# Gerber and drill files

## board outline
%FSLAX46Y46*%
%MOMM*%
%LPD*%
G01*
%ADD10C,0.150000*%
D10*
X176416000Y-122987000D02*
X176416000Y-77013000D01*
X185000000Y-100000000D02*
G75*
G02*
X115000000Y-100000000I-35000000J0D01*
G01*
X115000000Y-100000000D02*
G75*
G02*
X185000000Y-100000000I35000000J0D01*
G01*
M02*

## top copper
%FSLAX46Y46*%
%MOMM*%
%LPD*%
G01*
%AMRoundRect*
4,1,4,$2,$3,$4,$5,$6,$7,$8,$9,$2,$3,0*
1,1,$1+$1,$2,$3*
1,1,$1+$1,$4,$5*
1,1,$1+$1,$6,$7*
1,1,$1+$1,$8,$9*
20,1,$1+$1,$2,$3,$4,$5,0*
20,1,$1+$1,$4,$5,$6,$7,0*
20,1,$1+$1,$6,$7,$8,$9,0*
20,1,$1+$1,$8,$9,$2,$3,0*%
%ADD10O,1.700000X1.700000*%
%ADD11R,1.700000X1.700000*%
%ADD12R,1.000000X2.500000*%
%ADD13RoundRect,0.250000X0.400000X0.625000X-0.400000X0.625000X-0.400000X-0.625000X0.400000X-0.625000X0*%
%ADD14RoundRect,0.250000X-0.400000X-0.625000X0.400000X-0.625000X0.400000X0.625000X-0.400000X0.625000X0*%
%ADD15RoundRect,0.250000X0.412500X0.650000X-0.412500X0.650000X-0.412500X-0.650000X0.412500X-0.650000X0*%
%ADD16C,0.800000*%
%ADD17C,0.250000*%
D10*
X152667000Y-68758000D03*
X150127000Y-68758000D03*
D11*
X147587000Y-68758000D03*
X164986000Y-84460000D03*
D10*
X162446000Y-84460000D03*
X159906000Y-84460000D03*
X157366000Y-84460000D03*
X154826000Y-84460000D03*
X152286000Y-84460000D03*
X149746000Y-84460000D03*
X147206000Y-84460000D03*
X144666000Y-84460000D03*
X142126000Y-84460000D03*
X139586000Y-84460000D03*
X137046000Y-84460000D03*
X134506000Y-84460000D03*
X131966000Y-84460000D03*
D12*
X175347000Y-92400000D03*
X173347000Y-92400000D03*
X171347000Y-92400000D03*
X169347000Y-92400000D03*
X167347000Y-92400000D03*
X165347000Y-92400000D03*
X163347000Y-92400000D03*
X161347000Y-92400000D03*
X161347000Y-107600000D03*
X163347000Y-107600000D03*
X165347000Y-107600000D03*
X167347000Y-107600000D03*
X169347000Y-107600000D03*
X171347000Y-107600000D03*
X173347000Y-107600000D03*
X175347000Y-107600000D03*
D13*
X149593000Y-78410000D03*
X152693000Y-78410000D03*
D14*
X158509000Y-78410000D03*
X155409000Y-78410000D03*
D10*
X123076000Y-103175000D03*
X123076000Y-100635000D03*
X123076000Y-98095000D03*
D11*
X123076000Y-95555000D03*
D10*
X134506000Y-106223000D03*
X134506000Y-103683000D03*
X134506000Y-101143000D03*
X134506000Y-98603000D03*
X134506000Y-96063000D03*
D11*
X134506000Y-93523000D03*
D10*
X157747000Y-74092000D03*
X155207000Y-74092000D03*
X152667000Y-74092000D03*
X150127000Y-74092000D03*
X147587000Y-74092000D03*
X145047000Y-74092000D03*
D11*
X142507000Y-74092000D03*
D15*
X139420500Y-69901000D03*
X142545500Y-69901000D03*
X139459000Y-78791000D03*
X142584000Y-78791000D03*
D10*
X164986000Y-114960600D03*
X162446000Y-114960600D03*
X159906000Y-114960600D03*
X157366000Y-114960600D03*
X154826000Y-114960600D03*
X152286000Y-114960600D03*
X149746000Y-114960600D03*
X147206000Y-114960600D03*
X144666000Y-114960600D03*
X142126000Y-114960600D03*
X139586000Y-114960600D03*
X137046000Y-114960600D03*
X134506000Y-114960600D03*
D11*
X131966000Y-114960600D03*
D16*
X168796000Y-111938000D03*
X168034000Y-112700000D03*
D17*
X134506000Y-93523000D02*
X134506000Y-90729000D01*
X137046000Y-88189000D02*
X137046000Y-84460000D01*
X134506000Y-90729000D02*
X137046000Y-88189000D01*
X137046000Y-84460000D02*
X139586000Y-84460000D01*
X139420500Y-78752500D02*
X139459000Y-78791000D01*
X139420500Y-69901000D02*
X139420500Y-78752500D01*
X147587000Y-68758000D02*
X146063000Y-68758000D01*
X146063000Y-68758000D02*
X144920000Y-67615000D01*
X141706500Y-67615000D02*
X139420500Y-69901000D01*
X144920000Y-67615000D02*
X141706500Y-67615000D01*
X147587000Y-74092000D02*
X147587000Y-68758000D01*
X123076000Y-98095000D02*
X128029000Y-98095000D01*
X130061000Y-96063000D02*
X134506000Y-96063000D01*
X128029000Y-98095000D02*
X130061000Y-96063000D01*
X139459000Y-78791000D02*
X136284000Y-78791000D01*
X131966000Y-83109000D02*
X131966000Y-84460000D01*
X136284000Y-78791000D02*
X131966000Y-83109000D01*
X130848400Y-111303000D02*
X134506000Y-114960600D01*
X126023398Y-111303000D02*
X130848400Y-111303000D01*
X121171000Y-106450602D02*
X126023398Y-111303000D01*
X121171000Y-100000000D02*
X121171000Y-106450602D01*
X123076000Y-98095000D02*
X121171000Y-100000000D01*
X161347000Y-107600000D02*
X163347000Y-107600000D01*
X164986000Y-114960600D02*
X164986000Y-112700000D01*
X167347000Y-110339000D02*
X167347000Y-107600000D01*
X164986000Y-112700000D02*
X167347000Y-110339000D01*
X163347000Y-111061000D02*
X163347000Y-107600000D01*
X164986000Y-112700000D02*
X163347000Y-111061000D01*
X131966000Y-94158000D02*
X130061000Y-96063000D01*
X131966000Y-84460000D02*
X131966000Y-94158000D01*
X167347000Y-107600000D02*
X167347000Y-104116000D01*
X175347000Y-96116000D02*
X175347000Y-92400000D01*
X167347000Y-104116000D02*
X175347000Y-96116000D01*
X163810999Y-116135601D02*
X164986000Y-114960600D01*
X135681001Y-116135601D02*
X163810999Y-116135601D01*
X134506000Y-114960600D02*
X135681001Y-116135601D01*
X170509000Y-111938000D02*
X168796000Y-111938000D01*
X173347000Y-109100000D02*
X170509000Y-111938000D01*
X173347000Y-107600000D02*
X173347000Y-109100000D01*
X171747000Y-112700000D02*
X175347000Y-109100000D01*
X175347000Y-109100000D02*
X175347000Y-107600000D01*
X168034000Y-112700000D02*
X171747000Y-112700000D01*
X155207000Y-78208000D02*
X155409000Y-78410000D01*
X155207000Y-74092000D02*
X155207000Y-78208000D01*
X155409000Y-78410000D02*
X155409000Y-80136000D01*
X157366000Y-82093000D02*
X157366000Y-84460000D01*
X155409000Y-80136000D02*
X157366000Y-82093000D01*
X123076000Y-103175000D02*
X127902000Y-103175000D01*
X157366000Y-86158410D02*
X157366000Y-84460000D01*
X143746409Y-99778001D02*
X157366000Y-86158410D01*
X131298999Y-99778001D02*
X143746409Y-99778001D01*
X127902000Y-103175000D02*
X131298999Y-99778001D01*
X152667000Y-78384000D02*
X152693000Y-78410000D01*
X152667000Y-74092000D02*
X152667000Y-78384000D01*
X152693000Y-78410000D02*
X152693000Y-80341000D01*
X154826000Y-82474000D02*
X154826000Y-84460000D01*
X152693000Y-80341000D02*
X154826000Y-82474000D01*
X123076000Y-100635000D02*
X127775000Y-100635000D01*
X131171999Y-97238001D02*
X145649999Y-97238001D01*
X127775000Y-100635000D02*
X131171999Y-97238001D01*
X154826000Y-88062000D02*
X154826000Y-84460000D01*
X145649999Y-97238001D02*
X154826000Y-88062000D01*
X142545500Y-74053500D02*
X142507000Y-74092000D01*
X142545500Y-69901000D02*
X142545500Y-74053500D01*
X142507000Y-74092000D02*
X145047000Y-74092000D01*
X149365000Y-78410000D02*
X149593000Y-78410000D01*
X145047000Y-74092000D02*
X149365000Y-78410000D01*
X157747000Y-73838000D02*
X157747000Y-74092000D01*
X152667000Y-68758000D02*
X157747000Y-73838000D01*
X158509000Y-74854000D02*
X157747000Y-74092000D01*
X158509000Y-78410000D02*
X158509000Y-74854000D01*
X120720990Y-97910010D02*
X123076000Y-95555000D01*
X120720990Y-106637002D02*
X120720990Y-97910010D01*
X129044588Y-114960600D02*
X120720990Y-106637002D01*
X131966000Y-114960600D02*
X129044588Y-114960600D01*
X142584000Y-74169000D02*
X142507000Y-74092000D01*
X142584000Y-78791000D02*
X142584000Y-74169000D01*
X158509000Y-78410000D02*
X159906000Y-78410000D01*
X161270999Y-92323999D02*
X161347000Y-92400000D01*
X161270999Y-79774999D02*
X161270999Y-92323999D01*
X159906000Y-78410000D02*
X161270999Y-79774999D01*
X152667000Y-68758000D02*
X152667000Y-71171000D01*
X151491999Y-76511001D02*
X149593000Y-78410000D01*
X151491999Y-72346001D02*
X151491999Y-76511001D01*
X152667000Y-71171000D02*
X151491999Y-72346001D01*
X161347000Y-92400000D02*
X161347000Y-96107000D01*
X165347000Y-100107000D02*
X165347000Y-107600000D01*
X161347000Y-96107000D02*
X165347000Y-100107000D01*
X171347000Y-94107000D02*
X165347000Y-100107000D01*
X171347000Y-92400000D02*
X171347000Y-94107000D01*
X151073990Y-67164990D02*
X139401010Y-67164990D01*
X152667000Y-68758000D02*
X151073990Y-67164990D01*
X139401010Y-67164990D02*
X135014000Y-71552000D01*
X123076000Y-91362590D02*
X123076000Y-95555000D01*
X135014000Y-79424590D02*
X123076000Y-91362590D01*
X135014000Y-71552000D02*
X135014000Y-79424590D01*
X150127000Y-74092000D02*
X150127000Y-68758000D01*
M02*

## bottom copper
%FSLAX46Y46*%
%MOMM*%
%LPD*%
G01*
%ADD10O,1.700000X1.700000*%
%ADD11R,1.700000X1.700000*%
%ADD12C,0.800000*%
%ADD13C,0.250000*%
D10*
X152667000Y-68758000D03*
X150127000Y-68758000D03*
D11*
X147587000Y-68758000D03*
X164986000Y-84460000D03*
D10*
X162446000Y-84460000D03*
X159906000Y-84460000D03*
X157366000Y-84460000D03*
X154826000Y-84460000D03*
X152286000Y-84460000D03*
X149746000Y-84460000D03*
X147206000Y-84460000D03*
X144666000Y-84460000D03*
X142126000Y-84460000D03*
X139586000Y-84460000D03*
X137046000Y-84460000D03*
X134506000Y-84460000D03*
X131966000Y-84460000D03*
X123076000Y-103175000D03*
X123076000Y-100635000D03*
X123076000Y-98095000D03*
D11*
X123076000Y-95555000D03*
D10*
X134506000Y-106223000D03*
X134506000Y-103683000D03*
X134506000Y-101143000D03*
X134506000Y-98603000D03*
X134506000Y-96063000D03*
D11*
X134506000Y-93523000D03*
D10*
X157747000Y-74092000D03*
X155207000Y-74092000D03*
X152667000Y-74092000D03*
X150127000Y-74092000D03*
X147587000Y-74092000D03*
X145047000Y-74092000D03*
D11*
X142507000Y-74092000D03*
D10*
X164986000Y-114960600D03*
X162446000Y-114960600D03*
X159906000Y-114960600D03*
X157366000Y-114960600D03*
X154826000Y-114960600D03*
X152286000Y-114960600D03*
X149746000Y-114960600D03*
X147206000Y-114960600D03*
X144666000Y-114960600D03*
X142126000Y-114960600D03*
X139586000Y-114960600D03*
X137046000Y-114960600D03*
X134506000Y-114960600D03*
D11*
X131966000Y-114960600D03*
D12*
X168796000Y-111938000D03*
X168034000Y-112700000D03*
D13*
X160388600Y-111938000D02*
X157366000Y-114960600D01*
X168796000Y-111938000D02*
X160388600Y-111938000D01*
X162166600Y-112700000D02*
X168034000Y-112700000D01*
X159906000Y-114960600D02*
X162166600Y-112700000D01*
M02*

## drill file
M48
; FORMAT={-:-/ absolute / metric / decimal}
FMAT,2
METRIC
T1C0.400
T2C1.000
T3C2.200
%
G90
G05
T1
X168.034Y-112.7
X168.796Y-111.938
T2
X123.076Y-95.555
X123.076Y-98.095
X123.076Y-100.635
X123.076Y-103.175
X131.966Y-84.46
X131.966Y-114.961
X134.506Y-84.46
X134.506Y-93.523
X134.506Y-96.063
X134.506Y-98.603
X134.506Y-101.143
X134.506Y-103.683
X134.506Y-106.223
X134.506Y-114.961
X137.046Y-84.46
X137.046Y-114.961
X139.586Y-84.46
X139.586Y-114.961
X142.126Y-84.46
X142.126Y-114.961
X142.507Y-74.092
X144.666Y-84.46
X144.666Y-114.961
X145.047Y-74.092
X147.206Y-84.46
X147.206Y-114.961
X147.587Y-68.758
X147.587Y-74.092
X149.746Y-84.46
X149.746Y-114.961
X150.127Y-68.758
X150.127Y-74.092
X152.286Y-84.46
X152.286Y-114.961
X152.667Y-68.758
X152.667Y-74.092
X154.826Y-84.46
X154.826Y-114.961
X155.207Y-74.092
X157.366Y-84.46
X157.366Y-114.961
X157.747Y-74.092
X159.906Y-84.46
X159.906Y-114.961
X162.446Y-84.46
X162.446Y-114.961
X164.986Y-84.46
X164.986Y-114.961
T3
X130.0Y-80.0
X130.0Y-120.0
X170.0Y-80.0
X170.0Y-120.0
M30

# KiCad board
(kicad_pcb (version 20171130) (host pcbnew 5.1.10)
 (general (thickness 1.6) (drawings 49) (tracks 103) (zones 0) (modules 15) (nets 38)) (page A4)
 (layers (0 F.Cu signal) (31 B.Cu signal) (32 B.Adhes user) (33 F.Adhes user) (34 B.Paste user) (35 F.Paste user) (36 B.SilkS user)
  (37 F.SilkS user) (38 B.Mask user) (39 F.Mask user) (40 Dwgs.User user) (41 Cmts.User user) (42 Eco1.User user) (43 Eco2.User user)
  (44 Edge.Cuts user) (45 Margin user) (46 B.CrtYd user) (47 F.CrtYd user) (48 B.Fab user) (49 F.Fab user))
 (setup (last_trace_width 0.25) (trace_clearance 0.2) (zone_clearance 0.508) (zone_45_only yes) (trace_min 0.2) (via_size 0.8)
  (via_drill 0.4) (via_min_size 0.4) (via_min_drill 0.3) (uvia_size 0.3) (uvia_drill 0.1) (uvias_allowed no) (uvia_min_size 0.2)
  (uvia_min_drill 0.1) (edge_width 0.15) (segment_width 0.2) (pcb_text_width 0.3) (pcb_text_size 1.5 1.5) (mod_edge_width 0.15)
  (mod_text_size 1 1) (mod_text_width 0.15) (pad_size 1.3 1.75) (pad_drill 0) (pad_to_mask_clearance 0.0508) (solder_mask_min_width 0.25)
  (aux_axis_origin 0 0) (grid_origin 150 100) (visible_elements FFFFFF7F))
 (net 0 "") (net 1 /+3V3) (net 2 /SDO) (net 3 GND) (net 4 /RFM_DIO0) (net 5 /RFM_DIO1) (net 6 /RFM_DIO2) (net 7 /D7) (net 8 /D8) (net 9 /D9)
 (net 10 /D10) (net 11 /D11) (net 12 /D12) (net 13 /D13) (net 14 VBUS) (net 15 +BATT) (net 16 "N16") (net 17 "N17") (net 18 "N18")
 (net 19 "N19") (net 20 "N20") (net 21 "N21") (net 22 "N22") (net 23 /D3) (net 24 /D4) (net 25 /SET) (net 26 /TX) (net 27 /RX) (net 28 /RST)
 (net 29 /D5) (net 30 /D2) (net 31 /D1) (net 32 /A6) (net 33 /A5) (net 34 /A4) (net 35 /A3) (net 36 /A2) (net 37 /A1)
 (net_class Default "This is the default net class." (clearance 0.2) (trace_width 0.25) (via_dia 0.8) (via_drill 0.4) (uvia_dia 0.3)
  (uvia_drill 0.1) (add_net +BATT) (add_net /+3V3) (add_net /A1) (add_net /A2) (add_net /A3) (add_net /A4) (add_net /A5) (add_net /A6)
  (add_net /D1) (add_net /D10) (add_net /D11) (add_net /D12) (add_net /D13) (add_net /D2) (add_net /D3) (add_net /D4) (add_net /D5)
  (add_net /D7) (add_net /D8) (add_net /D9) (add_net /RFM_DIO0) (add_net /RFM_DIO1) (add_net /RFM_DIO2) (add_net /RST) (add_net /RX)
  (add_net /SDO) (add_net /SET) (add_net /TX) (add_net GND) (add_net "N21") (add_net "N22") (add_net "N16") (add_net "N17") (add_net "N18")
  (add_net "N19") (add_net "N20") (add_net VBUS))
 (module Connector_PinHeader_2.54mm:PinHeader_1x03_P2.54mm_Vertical (layer F.Cu) (at 147.587 68.758 90)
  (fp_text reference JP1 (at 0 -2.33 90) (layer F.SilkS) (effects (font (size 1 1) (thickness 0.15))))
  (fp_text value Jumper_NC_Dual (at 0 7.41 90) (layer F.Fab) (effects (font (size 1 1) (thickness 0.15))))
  (pad 3 thru_hole oval (at 0 5.08 90) (size 1.7 1.7) (drill 1) (layers *.Cu *.Mask) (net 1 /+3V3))
  (pad 2 thru_hole oval (at 0 2.54 90) (size 1.7 1.7) (drill 1) (layers *.Cu *.Mask) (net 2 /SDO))
  (pad 1 thru_hole rect (at 0 0 90) (size 1.7 1.7) (drill 1) (layers *.Cu *.Mask) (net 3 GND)))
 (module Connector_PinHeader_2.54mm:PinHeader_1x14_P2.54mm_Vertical (layer F.Cu) (at 164.986 84.46 270)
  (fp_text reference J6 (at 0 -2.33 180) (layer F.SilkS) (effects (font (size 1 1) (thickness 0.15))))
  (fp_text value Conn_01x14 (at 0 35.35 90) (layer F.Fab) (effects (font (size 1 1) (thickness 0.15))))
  (pad 1 thru_hole rect (at 0 0 270) (size 1.7 1.7) (drill 1) (layers *.Cu *.Mask) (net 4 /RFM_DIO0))
  (pad 2 thru_hole oval (at 0 2.54 270) (size 1.7 1.7) (drill 1) (layers *.Cu *.Mask) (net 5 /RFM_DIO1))
  (pad 3 thru_hole oval (at 0 5.08 270) (size 1.7 1.7) (drill 1) (layers *.Cu *.Mask) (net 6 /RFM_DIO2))
  (pad 4 thru_hole oval (at 0 7.62 270) (size 1.7 1.7) (drill 1) (layers *.Cu *.Mask) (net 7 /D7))
  (pad 5 thru_hole oval (at 0 10.16 270) (size 1.7 1.7) (drill 1) (layers *.Cu *.Mask) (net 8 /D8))
  (pad 6 thru_hole oval (at 0 12.7 270) (size 1.7 1.7) (drill 1) (layers *.Cu *.Mask) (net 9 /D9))
  (pad 7 thru_hole oval (at 0 15.24 270) (size 1.7 1.7) (drill 1) (layers *.Cu *.Mask) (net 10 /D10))
  (pad 8 thru_hole oval (at 0 17.78 270) (size 1.7 1.7) (drill 1) (layers *.Cu *.Mask) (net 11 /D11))
  (pad 9 thru_hole oval (at 0 20.32 270) (size 1.7 1.7) (drill 1) (layers *.Cu *.Mask) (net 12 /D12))
  (pad 10 thru_hole oval (at 0 22.86 270) (size 1.7 1.7) (drill 1) (layers *.Cu *.Mask) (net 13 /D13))
  (pad 11 thru_hole oval (at 0 25.4 270) (size 1.7 1.7) (drill 1) (layers *.Cu *.Mask) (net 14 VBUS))
  (pad 12 thru_hole oval (at 0 27.94 270) (size 1.7 1.7) (drill 1) (layers *.Cu *.Mask) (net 14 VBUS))
  (pad 13 thru_hole oval (at 0 30.48 270) (size 1.7 1.7) (drill 1) (layers *.Cu *.Mask) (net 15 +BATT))
  (pad 14 thru_hole oval (at 0 33.02 270) (size 1.7 1.7) (drill 1) (layers *.Cu *.Mask) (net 3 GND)))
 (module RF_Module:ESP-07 (layer F.Cu) (at 170.447 100 270)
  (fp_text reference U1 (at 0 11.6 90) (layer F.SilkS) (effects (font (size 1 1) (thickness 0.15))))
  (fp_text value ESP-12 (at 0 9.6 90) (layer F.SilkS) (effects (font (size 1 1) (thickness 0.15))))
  (pad 1 smd rect (at -7.6 -4.9 270) (size 2.5 1) (layers F.Cu F.Paste F.Mask) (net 3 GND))
  (pad 2 smd rect (at -7.6 -2.9 270) (size 2.5 1) (layers F.Cu F.Paste F.Mask) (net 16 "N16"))
  (pad 3 smd rect (at -7.6 -0.9 270) (size 2.5 1) (layers F.Cu F.Paste F.Mask) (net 1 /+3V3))
  (pad 4 smd rect (at -7.6 1.1 270) (size 2.5 1) (layers F.Cu F.Paste F.Mask) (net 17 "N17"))
  (pad 5 smd rect (at -7.6 3.1 270) (size 2.5 1) (layers F.Cu F.Paste F.Mask) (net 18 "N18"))
  (pad 6 smd rect (at -7.6 5.1 270) (size 2.5 1) (layers F.Cu F.Paste F.Mask) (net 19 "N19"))
  (pad 7 smd rect (at -7.6 7.1 270) (size 2.5 1) (layers F.Cu F.Paste F.Mask) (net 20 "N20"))
  (pad 8 smd rect (at -7.6 9.1 270) (size 2.5 1) (layers F.Cu F.Paste F.Mask) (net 1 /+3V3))
  (pad 9 smd rect (at 7.6 9.1 270) (size 2.5 1) (layers F.Cu F.Paste F.Mask) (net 3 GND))
  (pad 10 smd rect (at 7.6 7.1 270) (size 2.5 1) (layers F.Cu F.Paste F.Mask) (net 3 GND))
  (pad 11 smd rect (at 7.6 5.1 270) (size 2.5 1) (layers F.Cu F.Paste F.Mask) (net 1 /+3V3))
  (pad 12 smd rect (at 7.6 3.1 270) (size 2.5 1) (layers F.Cu F.Paste F.Mask) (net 3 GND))
  (pad 13 smd rect (at 7.6 1.1 270) (size 2.5 1) (layers F.Cu F.Paste F.Mask) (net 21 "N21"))
  (pad 14 smd rect (at 7.6 -0.9 270) (size 2.5 1) (layers F.Cu F.Paste F.Mask) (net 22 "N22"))
  (pad 15 smd rect (at 7.6 -2.9 270) (size 2.5 1) (layers F.Cu F.Paste F.Mask) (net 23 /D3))
  (pad 16 smd rect (at 7.6 -4.9 270) (size 2.5 1) (layers F.Cu F.Paste F.Mask) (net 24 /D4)))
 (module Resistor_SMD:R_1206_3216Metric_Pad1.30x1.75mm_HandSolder (layer F.Cu) (at 151.143 78.41 180)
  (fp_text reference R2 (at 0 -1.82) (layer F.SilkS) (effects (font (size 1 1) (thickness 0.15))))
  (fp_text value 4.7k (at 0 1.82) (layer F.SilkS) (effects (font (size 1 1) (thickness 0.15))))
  (pad 2 smd roundrect (at 1.55 0 180) (size 1.3 1.75) (layers F.Cu F.Paste F.Mask) (roundrect_rratio 0.192308) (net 1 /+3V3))
  (pad 1 smd roundrect (at -1.55 0 180) (size 1.3 1.75) (layers F.Cu F.Paste F.Mask) (roundrect_rratio 0.192308) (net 8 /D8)))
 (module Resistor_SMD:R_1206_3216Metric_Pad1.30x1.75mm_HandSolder (layer F.Cu) (at 156.959 78.41)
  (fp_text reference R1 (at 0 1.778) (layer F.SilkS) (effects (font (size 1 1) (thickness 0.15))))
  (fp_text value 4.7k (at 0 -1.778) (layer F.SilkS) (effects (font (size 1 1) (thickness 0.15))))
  (pad 2 smd roundrect (at 1.55 0) (size 1.3 1.75) (layers F.Cu F.Paste F.Mask) (roundrect_rratio 0.192308) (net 1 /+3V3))
  (pad 1 smd roundrect (at -1.55 0) (size 1.3 1.75) (layers F.Cu F.Paste F.Mask) (roundrect_rratio 0.192308) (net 7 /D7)))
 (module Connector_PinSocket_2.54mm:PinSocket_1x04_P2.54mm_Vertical (layer F.Cu) (at 123.076 95.555)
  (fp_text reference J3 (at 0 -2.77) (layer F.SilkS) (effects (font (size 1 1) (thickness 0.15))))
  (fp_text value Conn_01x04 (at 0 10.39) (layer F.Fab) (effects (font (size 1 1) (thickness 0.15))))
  (pad 4 thru_hole oval (at 0 7.62) (size 1.7 1.7) (drill 1) (layers *.Cu *.Mask) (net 7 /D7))
  (pad 3 thru_hole oval (at 0 5.08) (size 1.7 1.7) (drill 1) (layers *.Cu *.Mask) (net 8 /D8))
  (pad 2 thru_hole oval (at 0 2.54) (size 1.7 1.7) (drill 1) (layers *.Cu *.Mask) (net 3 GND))
  (pad 1 thru_hole rect (at 0 0) (size 1.7 1.7) (drill 1) (layers *.Cu *.Mask) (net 1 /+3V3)))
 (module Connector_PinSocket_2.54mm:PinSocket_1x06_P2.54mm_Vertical (layer F.Cu) (at 134.506 93.523)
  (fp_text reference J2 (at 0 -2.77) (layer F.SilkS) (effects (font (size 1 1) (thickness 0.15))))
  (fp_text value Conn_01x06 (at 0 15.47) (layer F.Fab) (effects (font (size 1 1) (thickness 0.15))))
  (pad 6 thru_hole oval (at 0 12.7) (size 1.7 1.7) (drill 1) (layers *.Cu *.Mask) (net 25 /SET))
  (pad 5 thru_hole oval (at 0 10.16) (size 1.7 1.7) (drill 1) (layers *.Cu *.Mask) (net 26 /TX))
  (pad 4 thru_hole oval (at 0 7.62) (size 1.7 1.7) (drill 1) (layers *.Cu *.Mask) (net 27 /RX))
  (pad 3 thru_hole oval (at 0 5.08) (size 1.7 1.7) (drill 1) (layers *.Cu *.Mask) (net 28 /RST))
  (pad 2 thru_hole oval (at 0 2.54) (size 1.7 1.7) (drill 1) (layers *.Cu *.Mask) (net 3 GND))
  (pad 1 thru_hole rect (at 0 0) (size 1.7 1.7) (drill 1) (layers *.Cu *.Mask) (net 14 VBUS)))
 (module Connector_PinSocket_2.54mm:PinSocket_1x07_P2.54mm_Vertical (layer F.Cu) (at 142.507 74.092 90)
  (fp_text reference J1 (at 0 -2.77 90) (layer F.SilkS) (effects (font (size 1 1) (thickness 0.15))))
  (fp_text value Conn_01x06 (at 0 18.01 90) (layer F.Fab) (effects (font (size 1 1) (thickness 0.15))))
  (pad 7 thru_hole oval (at 0 15.24 90) (size 1.7 1.7) (drill 1) (layers *.Cu *.Mask) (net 1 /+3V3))
  (pad 6 thru_hole oval (at 0 12.7 90) (size 1.7 1.7) (drill 1) (layers *.Cu *.Mask) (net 7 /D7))
  (pad 5 thru_hole oval (at 0 10.16 90) (size 1.7 1.7) (drill 1) (layers *.Cu *.Mask) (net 8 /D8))
  (pad 4 thru_hole oval (at 0 7.62 90) (size 1.7 1.7) (drill 1) (layers *.Cu *.Mask) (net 2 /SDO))
  (pad 3 thru_hole oval (at 0 5.08 90) (size 1.7 1.7) (drill 1) (layers *.Cu *.Mask) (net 3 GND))
  (pad 2 thru_hole oval (at 0 2.54 90) (size 1.7 1.7) (drill 1) (layers *.Cu *.Mask) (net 1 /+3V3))
  (pad 1 thru_hole rect (at 0 0 90) (size 1.7 1.7) (drill 1) (layers *.Cu *.Mask) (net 1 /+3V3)))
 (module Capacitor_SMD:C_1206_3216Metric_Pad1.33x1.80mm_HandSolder (layer F.Cu) (at 140.983 69.901 180)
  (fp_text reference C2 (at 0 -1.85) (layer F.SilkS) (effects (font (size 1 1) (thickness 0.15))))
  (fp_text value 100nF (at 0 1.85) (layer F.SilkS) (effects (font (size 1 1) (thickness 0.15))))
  (pad 2 smd roundrect (at 1.5625 0 180) (size 1.325 1.8) (layers F.Cu F.Paste F.Mask) (roundrect_rratio 0.188679) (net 3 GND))
  (pad 1 smd roundrect (at -1.5625 0 180) (size 1.325 1.8) (layers F.Cu F.Paste F.Mask) (roundrect_rratio 0.188679) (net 1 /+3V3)))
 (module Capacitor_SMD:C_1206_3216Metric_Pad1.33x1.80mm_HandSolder (layer F.Cu) (at 141.0215 78.791 180)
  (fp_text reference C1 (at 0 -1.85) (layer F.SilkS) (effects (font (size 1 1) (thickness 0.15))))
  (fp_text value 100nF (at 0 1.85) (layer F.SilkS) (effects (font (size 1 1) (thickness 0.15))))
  (pad 2 smd roundrect (at 1.5625 0 180) (size 1.325 1.8) (layers F.Cu F.Paste F.Mask) (roundrect_rratio 0.188679) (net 3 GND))
  (pad 1 smd roundrect (at -1.5625 0 180) (size 1.325 1.8) (layers F.Cu F.Paste F.Mask) (roundrect_rratio 0.188679) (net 1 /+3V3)))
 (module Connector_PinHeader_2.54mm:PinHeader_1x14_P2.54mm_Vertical (layer F.Cu) (at 131.966 114.9606 90)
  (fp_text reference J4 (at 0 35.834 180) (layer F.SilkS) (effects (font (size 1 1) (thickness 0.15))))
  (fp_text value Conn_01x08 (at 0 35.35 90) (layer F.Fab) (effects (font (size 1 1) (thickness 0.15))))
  (pad 14 thru_hole oval (at 0 33.02 90) (size 1.7 1.7) (drill 1) (layers *.Cu *.Mask) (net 3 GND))
  (pad 13 thru_hole oval (at 0 30.48 90) (size 1.7 1.7) (drill 1) (layers *.Cu *.Mask) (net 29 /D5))
  (pad 12 thru_hole oval (at 0 27.94 90) (size 1.7 1.7) (drill 1) (layers *.Cu *.Mask) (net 24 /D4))
  (pad 11 thru_hole oval (at 0 25.4 90) (size 1.7 1.7) (drill 1) (layers *.Cu *.Mask) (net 23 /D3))
  (pad 10 thru_hole oval (at 0 22.86 90) (size 1.7 1.7) (drill 1) (layers *.Cu *.Mask) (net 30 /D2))
  (pad 9 thru_hole oval (at 0 20.32 90) (size 1.7 1.7) (drill 1) (layers *.Cu *.Mask) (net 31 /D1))
  (pad 8 thru_hole oval (at 0 17.78 90) (size 1.7 1.7) (drill 1) (layers *.Cu *.Mask) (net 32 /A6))
  (pad 7 thru_hole oval (at 0 15.24 90) (size 1.7 1.7) (drill 1) (layers *.Cu *.Mask) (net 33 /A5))
  (pad 6 thru_hole oval (at 0 12.7 90) (size 1.7 1.7) (drill 1) (layers *.Cu *.Mask) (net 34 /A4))
  (pad 5 thru_hole oval (at 0 10.16 90) (size 1.7 1.7) (drill 1) (layers *.Cu *.Mask) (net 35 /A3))
  (pad 4 thru_hole oval (at 0 7.62 90) (size 1.7 1.7) (drill 1) (layers *.Cu *.Mask) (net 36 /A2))
  (pad 3 thru_hole oval (at 0 5.08 90) (size 1.7 1.7) (drill 1) (layers *.Cu *.Mask) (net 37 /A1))
  (pad 2 thru_hole oval (at 0 2.54 90) (size 1.7 1.7) (drill 1) (layers *.Cu *.Mask) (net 3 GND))
  (pad 1 thru_hole rect (at 0 0 90) (size 1.7 1.7) (drill 1) (layers *.Cu *.Mask) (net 1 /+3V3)))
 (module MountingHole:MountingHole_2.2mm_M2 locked (layer F.Cu) (at 130 120)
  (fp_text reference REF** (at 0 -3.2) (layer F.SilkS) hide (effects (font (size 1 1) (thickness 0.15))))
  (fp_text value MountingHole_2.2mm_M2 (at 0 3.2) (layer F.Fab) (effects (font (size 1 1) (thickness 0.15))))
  (pad 1 np_thru_hole circle (at 0 0) (size 2.2 2.2) (drill 2.2) (layers *.Cu *.Mask)))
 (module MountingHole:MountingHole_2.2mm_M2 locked (layer F.Cu) (at 170 120)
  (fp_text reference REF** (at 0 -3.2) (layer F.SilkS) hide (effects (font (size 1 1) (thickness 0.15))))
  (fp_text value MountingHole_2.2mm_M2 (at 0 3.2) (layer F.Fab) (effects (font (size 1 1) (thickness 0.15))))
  (pad 1 np_thru_hole circle (at 0 0) (size 2.2 2.2) (drill 2.2) (layers *.Cu *.Mask)))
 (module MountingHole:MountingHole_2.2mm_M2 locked (layer F.Cu) (at 130 80)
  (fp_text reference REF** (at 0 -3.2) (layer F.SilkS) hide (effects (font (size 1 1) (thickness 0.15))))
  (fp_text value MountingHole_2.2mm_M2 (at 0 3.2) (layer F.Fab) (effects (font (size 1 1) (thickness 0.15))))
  (pad 1 np_thru_hole circle (at 0 0) (size 2.2 2.2) (drill 2.2) (layers *.Cu *.Mask)))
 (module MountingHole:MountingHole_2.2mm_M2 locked (layer F.Cu) (at 170 80)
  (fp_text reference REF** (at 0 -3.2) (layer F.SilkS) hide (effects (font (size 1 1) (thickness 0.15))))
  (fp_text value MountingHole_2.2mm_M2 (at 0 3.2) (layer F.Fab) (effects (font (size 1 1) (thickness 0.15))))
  (pad 1 np_thru_hole circle (at 0 0) (size 2.2 2.2) (drill 2.2) (layers *.Cu *.Mask)))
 (gr_line (start 176.416 122.987) (end 176.416 77.013) (layer Edge.Cuts) (width 0.15))
 (gr_circle (center 150 100) (end 185 100) (layer Edge.Cuts) (width 0.15))
 (segment (start 134.506 93.523) (end 134.506 90.729) (width 0.25) (layer F.Cu) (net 14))
 (segment (start 137.046 88.189) (end 137.046 84.46) (width 0.25) (layer F.Cu) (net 14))
 (segment (start 134.506 90.729) (end 137.046 88.189) (width 0.25) (layer F.Cu) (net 14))
 (segment (start 137.046 84.46) (end 139.586 84.46) (width 0.25) (layer F.Cu) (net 14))
 (segment (start 139.4205 78.7525) (end 139.459 78.791) (width 0.25) (layer F.Cu) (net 3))
 (segment (start 139.4205 69.901) (end 139.4205 78.7525) (width 0.25) (layer F.Cu) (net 3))
 (segment (start 147.587 68.758) (end 146.063 68.758) (width 0.25) (layer F.Cu) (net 3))
 (segment (start 146.063 68.758) (end 144.92 67.615) (width 0.25) (layer F.Cu) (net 3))
 (segment (start 141.7065 67.615) (end 139.4205 69.901) (width 0.25) (layer F.Cu) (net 3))
 (segment (start 144.92 67.615) (end 141.7065 67.615) (width 0.25) (layer F.Cu) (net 3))
 (segment (start 147.587 74.092) (end 147.587 68.758) (width 0.25) (layer F.Cu) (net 3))
 (segment (start 123.076 98.095) (end 128.029 98.095) (width 0.25) (layer F.Cu) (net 3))
 (segment (start 130.061 96.063) (end 134.506 96.063) (width 0.25) (layer F.Cu) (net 3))
 (segment (start 128.029 98.095) (end 130.061 96.063) (width 0.25) (layer F.Cu) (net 3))
 (segment (start 139.459 78.791) (end 136.284 78.791) (width 0.25) (layer F.Cu) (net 3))
 (segment (start 131.966 83.109) (end 131.966 84.46) (width 0.25) (layer F.Cu) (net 3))
 (segment (start 136.284 78.791) (end 131.966 83.109) (width 0.25) (layer F.Cu) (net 3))
 (segment (start 130.8484 111.303) (end 134.506 114.9606) (width 0.25) (layer F.Cu) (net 3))
 (segment (start 126.023398 111.303) (end 130.8484 111.303) (width 0.25) (layer F.Cu) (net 3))
 (segment (start 121.171 106.450602) (end 126.023398 111.303) (width 0.25) (layer F.Cu) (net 3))
 (segment (start 121.171 100) (end 121.171 106.450602) (width 0.25) (layer F.Cu) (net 3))
 (segment (start 123.076 98.095) (end 121.171 100) (width 0.25) (layer F.Cu) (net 3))
 (segment (start 161.347 107.6) (end 163.347 107.6) (width 0.25) (layer F.Cu) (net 3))
 (segment (start 164.986 114.9606) (end 164.986 112.7) (width 0.25) (layer F.Cu) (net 3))
 (segment (start 167.347 110.339) (end 167.347 107.6) (width 0.25) (layer F.Cu) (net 3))
 (segment (start 164.986 112.7) (end 167.347 110.339) (width 0.25) (layer F.Cu) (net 3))
 (segment (start 163.347 111.061) (end 163.347 107.6) (width 0.25) (layer F.Cu) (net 3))
 (segment (start 164.986 112.7) (end 163.347 111.061) (width 0.25) (layer F.Cu) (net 3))
 (segment (start 131.966 94.158) (end 130.061 96.063) (width 0.25) (layer F.Cu) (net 3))
 (segment (start 131.966 84.46) (end 131.966 94.158) (width 0.25) (layer F.Cu) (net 3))
 (segment (start 167.347 107.6) (end 167.347 104.116) (width 0.25) (layer F.Cu) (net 3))
 (segment (start 175.347 96.116) (end 175.347 92.4) (width 0.25) (layer F.Cu) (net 3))
 (segment (start 167.347 104.116) (end 175.347 96.116) (width 0.25) (layer F.Cu) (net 3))
 (segment (start 163.810999 116.135601) (end 164.986 114.9606) (width 0.25) (layer F.Cu) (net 3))
 (segment (start 135.681001 116.135601) (end 163.810999 116.135601) (width 0.25) (layer F.Cu) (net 3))
 (segment (start 134.506 114.9606) (end 135.681001 116.135601) (width 0.25) (layer F.Cu) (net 3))
 (via (at 168.796 111.938) (size 0.8) (drill 0.4) (layers F.Cu B.Cu) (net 23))
 (segment (start 170.509 111.938) (end 168.796 111.938) (width 0.25) (layer F.Cu) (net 23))
 (segment (start 173.347 109.1) (end 170.509 111.938) (width 0.25) (layer F.Cu) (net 23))
 (segment (start 173.347 107.6) (end 173.347 109.1) (width 0.25) (layer F.Cu) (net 23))
 (segment (start 160.3886 111.938) (end 157.366 114.9606) (width 0.25) (layer B.Cu) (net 23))
 (segment (start 168.796 111.938) (end 160.3886 111.938) (width 0.25) (layer B.Cu) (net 23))
 (via (at 168.034 112.7) (size 0.8) (drill 0.4) (layers F.Cu B.Cu) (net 24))
 (segment (start 162.1666 112.7) (end 168.034 112.7) (width 0.25) (layer B.Cu) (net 24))
 (segment (start 159.906 114.9606) (end 162.1666 112.7) (width 0.25) (layer B.Cu) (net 24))
 (segment (start 171.747 112.7) (end 175.347 109.1) (width 0.25) (layer F.Cu) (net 24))
 (segment (start 175.347 109.1) (end 175.347 107.6) (width 0.25) (layer F.Cu) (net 24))
 (segment (start 168.034 112.7) (end 171.747 112.7) (width 0.25) (layer F.Cu) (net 24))
 (segment (start 155.207 78.208) (end 155.409 78.41) (width 0.25) (layer F.Cu) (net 7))
 (segment (start 155.207 74.092) (end 155.207 78.208) (width 0.25) (layer F.Cu) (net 7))
 (segment (start 155.409 78.41) (end 155.409 80.136) (width 0.25) (layer F.Cu) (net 7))
 (segment (start 157.366 82.093) (end 157.366 84.46) (width 0.25) (layer F.Cu) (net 7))
 (segment (start 155.409 80.136) (end 157.366 82.093) (width 0.25) (layer F.Cu) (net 7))
 (segment (start 123.076 103.175) (end 127.902 103.175) (width 0.25) (layer F.Cu) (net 7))
 (segment (start 157.366 86.15841) (end 157.366 84.46) (width 0.25) (layer F.Cu) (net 7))
 (segment (start 143.746409 99.778001) (end 157.366 86.15841) (width 0.25) (layer F.Cu) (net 7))
 (segment (start 131.298999 99.778001) (end 143.746409 99.778001) (width 0.25) (layer F.Cu) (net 7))
 (segment (start 127.902 103.175) (end 131.298999 99.778001) (width 0.25) (layer F.Cu) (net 7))
 (segment (start 152.667 78.384) (end 152.693 78.41) (width 0.25) (layer F.Cu) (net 8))
 (segment (start 152.667 74.092) (end 152.667 78.384) (width 0.25) (layer F.Cu) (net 8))
 (segment (start 152.693 78.41) (end 152.693 80.341) (width 0.25) (layer F.Cu) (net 8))
 (segment (start 154.826 82.474) (end 154.826 84.46) (width 0.25) (layer F.Cu) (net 8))
 (segment (start 152.693 80.341) (end 154.826 82.474) (width 0.25) (layer F.Cu) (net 8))
 (segment (start 123.076 100.635) (end 127.775 100.635) (width 0.25) (layer F.Cu) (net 8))
 (segment (start 131.171999 97.238001) (end 145.649999 97.238001) (width 0.25) (layer F.Cu) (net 8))
 (segment (start 127.775 100.635) (end 131.171999 97.238001) (width 0.25) (layer F.Cu) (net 8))
 (segment (start 154.826 88.062) (end 154.826 84.46) (width 0.25) (layer F.Cu) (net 8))
 (segment (start 145.649999 97.238001) (end 154.826 88.062) (width 0.25) (layer F.Cu) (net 8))
 (segment (start 142.5455 74.0535) (end 142.507 74.092) (width 0.25) (layer F.Cu) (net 1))
 (segment (start 142.5455 69.901) (end 142.5455 74.0535) (width 0.25) (layer F.Cu) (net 1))
 (segment (start 142.507 74.092) (end 145.047 74.092) (width 0.25) (layer F.Cu) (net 1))
 (segment (start 149.365 78.41) (end 149.593 78.41) (width 0.25) (layer F.Cu) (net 1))
 (segment (start 145.047 74.092) (end 149.365 78.41) (width 0.25) (layer F.Cu) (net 1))
 (segment (start 157.747 73.838) (end 157.747 74.092) (width 0.25) (layer F.Cu) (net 1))
 (segment (start 152.667 68.758) (end 157.747 73.838) (width 0.25) (layer F.Cu) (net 1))
 (segment (start 158.509 74.854) (end 157.747 74.092) (width 0.25) (layer F.Cu) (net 1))
 (segment (start 158.509 78.41) (end 158.509 74.854) (width 0.25) (layer F.Cu) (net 1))
 (segment (start 120.72099 97.91001) (end 123.076 95.555) (width 0.25) (layer F.Cu) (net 1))
 (segment (start 120.72099 106.637002) (end 120.72099 97.91001) (width 0.25) (layer F.Cu) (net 1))
 (segment (start 129.044588 114.9606) (end 120.72099 106.637002) (width 0.25) (layer F.Cu) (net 1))
 (segment (start 131.966 114.9606) (end 129.044588 114.9606) (width 0.25) (layer F.Cu) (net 1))
 (segment (start 142.584 74.169) (end 142.507 74.092) (width 0.25) (layer F.Cu) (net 1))
 (segment (start 142.584 78.791) (end 142.584 74.169) (width 0.25) (layer F.Cu) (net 1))
 (segment (start 158.509 78.41) (end 159.906 78.41) (width 0.25) (layer F.Cu) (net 1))
 (segment (start 161.270999 92.323999) (end 161.347 92.4) (width 0.25) (layer F.Cu) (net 1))
 (segment (start 161.270999 79.774999) (end 161.270999 92.323999) (width 0.25) (layer F.Cu) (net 1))
 (segment (start 159.906 78.41) (end 161.270999 79.774999) (width 0.25) (layer F.Cu) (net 1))
 (segment (start 152.667 68.758) (end 152.667 71.171) (width 0.25) (layer F.Cu) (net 1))
 (segment (start 151.491999 76.511001) (end 149.593 78.41) (width 0.25) (layer F.Cu) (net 1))
 (segment (start 151.491999 72.346001) (end 151.491999 76.511001) (width 0.25) (layer F.Cu) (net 1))
 (segment (start 152.667 71.171) (end 151.491999 72.346001) (width 0.25) (layer F.Cu) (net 1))
 (segment (start 161.347 92.4) (end 161.347 96.107) (width 0.25) (layer F.Cu) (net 1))
 (segment (start 165.347 100.107) (end 165.347 107.6) (width 0.25) (layer F.Cu) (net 1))
 (segment (start 161.347 96.107) (end 165.347 100.107) (width 0.25) (layer F.Cu) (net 1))
 (segment (start 171.347 94.107) (end 165.347 100.107) (width 0.25) (layer F.Cu) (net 1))
 (segment (start 171.347 92.4) (end 171.347 94.107) (width 0.25) (layer F.Cu) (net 1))
 (segment (start 151.07399 67.16499) (end 139.40101 67.16499) (width 0.25) (layer F.Cu) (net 1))
 (segment (start 152.667 68.758) (end 151.07399 67.16499) (width 0.25) (layer F.Cu) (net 1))
 (segment (start 139.40101 67.16499) (end 135.014 71.552) (width 0.25) (layer F.Cu) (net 1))
 (segment (start 123.076 91.36259) (end 123.076 95.555) (width 0.25) (layer F.Cu) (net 1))
 (segment (start 135.014 79.42459) (end 123.076 91.36259) (width 0.25) (layer F.Cu) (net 1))
 (segment (start 135.014 71.552) (end 135.014 79.42459) (width 0.25) (layer F.Cu) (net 1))
 (segment (start 150.127 74.092) (end 150.127 68.758) (width 0.25) (layer F.Cu) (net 2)))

